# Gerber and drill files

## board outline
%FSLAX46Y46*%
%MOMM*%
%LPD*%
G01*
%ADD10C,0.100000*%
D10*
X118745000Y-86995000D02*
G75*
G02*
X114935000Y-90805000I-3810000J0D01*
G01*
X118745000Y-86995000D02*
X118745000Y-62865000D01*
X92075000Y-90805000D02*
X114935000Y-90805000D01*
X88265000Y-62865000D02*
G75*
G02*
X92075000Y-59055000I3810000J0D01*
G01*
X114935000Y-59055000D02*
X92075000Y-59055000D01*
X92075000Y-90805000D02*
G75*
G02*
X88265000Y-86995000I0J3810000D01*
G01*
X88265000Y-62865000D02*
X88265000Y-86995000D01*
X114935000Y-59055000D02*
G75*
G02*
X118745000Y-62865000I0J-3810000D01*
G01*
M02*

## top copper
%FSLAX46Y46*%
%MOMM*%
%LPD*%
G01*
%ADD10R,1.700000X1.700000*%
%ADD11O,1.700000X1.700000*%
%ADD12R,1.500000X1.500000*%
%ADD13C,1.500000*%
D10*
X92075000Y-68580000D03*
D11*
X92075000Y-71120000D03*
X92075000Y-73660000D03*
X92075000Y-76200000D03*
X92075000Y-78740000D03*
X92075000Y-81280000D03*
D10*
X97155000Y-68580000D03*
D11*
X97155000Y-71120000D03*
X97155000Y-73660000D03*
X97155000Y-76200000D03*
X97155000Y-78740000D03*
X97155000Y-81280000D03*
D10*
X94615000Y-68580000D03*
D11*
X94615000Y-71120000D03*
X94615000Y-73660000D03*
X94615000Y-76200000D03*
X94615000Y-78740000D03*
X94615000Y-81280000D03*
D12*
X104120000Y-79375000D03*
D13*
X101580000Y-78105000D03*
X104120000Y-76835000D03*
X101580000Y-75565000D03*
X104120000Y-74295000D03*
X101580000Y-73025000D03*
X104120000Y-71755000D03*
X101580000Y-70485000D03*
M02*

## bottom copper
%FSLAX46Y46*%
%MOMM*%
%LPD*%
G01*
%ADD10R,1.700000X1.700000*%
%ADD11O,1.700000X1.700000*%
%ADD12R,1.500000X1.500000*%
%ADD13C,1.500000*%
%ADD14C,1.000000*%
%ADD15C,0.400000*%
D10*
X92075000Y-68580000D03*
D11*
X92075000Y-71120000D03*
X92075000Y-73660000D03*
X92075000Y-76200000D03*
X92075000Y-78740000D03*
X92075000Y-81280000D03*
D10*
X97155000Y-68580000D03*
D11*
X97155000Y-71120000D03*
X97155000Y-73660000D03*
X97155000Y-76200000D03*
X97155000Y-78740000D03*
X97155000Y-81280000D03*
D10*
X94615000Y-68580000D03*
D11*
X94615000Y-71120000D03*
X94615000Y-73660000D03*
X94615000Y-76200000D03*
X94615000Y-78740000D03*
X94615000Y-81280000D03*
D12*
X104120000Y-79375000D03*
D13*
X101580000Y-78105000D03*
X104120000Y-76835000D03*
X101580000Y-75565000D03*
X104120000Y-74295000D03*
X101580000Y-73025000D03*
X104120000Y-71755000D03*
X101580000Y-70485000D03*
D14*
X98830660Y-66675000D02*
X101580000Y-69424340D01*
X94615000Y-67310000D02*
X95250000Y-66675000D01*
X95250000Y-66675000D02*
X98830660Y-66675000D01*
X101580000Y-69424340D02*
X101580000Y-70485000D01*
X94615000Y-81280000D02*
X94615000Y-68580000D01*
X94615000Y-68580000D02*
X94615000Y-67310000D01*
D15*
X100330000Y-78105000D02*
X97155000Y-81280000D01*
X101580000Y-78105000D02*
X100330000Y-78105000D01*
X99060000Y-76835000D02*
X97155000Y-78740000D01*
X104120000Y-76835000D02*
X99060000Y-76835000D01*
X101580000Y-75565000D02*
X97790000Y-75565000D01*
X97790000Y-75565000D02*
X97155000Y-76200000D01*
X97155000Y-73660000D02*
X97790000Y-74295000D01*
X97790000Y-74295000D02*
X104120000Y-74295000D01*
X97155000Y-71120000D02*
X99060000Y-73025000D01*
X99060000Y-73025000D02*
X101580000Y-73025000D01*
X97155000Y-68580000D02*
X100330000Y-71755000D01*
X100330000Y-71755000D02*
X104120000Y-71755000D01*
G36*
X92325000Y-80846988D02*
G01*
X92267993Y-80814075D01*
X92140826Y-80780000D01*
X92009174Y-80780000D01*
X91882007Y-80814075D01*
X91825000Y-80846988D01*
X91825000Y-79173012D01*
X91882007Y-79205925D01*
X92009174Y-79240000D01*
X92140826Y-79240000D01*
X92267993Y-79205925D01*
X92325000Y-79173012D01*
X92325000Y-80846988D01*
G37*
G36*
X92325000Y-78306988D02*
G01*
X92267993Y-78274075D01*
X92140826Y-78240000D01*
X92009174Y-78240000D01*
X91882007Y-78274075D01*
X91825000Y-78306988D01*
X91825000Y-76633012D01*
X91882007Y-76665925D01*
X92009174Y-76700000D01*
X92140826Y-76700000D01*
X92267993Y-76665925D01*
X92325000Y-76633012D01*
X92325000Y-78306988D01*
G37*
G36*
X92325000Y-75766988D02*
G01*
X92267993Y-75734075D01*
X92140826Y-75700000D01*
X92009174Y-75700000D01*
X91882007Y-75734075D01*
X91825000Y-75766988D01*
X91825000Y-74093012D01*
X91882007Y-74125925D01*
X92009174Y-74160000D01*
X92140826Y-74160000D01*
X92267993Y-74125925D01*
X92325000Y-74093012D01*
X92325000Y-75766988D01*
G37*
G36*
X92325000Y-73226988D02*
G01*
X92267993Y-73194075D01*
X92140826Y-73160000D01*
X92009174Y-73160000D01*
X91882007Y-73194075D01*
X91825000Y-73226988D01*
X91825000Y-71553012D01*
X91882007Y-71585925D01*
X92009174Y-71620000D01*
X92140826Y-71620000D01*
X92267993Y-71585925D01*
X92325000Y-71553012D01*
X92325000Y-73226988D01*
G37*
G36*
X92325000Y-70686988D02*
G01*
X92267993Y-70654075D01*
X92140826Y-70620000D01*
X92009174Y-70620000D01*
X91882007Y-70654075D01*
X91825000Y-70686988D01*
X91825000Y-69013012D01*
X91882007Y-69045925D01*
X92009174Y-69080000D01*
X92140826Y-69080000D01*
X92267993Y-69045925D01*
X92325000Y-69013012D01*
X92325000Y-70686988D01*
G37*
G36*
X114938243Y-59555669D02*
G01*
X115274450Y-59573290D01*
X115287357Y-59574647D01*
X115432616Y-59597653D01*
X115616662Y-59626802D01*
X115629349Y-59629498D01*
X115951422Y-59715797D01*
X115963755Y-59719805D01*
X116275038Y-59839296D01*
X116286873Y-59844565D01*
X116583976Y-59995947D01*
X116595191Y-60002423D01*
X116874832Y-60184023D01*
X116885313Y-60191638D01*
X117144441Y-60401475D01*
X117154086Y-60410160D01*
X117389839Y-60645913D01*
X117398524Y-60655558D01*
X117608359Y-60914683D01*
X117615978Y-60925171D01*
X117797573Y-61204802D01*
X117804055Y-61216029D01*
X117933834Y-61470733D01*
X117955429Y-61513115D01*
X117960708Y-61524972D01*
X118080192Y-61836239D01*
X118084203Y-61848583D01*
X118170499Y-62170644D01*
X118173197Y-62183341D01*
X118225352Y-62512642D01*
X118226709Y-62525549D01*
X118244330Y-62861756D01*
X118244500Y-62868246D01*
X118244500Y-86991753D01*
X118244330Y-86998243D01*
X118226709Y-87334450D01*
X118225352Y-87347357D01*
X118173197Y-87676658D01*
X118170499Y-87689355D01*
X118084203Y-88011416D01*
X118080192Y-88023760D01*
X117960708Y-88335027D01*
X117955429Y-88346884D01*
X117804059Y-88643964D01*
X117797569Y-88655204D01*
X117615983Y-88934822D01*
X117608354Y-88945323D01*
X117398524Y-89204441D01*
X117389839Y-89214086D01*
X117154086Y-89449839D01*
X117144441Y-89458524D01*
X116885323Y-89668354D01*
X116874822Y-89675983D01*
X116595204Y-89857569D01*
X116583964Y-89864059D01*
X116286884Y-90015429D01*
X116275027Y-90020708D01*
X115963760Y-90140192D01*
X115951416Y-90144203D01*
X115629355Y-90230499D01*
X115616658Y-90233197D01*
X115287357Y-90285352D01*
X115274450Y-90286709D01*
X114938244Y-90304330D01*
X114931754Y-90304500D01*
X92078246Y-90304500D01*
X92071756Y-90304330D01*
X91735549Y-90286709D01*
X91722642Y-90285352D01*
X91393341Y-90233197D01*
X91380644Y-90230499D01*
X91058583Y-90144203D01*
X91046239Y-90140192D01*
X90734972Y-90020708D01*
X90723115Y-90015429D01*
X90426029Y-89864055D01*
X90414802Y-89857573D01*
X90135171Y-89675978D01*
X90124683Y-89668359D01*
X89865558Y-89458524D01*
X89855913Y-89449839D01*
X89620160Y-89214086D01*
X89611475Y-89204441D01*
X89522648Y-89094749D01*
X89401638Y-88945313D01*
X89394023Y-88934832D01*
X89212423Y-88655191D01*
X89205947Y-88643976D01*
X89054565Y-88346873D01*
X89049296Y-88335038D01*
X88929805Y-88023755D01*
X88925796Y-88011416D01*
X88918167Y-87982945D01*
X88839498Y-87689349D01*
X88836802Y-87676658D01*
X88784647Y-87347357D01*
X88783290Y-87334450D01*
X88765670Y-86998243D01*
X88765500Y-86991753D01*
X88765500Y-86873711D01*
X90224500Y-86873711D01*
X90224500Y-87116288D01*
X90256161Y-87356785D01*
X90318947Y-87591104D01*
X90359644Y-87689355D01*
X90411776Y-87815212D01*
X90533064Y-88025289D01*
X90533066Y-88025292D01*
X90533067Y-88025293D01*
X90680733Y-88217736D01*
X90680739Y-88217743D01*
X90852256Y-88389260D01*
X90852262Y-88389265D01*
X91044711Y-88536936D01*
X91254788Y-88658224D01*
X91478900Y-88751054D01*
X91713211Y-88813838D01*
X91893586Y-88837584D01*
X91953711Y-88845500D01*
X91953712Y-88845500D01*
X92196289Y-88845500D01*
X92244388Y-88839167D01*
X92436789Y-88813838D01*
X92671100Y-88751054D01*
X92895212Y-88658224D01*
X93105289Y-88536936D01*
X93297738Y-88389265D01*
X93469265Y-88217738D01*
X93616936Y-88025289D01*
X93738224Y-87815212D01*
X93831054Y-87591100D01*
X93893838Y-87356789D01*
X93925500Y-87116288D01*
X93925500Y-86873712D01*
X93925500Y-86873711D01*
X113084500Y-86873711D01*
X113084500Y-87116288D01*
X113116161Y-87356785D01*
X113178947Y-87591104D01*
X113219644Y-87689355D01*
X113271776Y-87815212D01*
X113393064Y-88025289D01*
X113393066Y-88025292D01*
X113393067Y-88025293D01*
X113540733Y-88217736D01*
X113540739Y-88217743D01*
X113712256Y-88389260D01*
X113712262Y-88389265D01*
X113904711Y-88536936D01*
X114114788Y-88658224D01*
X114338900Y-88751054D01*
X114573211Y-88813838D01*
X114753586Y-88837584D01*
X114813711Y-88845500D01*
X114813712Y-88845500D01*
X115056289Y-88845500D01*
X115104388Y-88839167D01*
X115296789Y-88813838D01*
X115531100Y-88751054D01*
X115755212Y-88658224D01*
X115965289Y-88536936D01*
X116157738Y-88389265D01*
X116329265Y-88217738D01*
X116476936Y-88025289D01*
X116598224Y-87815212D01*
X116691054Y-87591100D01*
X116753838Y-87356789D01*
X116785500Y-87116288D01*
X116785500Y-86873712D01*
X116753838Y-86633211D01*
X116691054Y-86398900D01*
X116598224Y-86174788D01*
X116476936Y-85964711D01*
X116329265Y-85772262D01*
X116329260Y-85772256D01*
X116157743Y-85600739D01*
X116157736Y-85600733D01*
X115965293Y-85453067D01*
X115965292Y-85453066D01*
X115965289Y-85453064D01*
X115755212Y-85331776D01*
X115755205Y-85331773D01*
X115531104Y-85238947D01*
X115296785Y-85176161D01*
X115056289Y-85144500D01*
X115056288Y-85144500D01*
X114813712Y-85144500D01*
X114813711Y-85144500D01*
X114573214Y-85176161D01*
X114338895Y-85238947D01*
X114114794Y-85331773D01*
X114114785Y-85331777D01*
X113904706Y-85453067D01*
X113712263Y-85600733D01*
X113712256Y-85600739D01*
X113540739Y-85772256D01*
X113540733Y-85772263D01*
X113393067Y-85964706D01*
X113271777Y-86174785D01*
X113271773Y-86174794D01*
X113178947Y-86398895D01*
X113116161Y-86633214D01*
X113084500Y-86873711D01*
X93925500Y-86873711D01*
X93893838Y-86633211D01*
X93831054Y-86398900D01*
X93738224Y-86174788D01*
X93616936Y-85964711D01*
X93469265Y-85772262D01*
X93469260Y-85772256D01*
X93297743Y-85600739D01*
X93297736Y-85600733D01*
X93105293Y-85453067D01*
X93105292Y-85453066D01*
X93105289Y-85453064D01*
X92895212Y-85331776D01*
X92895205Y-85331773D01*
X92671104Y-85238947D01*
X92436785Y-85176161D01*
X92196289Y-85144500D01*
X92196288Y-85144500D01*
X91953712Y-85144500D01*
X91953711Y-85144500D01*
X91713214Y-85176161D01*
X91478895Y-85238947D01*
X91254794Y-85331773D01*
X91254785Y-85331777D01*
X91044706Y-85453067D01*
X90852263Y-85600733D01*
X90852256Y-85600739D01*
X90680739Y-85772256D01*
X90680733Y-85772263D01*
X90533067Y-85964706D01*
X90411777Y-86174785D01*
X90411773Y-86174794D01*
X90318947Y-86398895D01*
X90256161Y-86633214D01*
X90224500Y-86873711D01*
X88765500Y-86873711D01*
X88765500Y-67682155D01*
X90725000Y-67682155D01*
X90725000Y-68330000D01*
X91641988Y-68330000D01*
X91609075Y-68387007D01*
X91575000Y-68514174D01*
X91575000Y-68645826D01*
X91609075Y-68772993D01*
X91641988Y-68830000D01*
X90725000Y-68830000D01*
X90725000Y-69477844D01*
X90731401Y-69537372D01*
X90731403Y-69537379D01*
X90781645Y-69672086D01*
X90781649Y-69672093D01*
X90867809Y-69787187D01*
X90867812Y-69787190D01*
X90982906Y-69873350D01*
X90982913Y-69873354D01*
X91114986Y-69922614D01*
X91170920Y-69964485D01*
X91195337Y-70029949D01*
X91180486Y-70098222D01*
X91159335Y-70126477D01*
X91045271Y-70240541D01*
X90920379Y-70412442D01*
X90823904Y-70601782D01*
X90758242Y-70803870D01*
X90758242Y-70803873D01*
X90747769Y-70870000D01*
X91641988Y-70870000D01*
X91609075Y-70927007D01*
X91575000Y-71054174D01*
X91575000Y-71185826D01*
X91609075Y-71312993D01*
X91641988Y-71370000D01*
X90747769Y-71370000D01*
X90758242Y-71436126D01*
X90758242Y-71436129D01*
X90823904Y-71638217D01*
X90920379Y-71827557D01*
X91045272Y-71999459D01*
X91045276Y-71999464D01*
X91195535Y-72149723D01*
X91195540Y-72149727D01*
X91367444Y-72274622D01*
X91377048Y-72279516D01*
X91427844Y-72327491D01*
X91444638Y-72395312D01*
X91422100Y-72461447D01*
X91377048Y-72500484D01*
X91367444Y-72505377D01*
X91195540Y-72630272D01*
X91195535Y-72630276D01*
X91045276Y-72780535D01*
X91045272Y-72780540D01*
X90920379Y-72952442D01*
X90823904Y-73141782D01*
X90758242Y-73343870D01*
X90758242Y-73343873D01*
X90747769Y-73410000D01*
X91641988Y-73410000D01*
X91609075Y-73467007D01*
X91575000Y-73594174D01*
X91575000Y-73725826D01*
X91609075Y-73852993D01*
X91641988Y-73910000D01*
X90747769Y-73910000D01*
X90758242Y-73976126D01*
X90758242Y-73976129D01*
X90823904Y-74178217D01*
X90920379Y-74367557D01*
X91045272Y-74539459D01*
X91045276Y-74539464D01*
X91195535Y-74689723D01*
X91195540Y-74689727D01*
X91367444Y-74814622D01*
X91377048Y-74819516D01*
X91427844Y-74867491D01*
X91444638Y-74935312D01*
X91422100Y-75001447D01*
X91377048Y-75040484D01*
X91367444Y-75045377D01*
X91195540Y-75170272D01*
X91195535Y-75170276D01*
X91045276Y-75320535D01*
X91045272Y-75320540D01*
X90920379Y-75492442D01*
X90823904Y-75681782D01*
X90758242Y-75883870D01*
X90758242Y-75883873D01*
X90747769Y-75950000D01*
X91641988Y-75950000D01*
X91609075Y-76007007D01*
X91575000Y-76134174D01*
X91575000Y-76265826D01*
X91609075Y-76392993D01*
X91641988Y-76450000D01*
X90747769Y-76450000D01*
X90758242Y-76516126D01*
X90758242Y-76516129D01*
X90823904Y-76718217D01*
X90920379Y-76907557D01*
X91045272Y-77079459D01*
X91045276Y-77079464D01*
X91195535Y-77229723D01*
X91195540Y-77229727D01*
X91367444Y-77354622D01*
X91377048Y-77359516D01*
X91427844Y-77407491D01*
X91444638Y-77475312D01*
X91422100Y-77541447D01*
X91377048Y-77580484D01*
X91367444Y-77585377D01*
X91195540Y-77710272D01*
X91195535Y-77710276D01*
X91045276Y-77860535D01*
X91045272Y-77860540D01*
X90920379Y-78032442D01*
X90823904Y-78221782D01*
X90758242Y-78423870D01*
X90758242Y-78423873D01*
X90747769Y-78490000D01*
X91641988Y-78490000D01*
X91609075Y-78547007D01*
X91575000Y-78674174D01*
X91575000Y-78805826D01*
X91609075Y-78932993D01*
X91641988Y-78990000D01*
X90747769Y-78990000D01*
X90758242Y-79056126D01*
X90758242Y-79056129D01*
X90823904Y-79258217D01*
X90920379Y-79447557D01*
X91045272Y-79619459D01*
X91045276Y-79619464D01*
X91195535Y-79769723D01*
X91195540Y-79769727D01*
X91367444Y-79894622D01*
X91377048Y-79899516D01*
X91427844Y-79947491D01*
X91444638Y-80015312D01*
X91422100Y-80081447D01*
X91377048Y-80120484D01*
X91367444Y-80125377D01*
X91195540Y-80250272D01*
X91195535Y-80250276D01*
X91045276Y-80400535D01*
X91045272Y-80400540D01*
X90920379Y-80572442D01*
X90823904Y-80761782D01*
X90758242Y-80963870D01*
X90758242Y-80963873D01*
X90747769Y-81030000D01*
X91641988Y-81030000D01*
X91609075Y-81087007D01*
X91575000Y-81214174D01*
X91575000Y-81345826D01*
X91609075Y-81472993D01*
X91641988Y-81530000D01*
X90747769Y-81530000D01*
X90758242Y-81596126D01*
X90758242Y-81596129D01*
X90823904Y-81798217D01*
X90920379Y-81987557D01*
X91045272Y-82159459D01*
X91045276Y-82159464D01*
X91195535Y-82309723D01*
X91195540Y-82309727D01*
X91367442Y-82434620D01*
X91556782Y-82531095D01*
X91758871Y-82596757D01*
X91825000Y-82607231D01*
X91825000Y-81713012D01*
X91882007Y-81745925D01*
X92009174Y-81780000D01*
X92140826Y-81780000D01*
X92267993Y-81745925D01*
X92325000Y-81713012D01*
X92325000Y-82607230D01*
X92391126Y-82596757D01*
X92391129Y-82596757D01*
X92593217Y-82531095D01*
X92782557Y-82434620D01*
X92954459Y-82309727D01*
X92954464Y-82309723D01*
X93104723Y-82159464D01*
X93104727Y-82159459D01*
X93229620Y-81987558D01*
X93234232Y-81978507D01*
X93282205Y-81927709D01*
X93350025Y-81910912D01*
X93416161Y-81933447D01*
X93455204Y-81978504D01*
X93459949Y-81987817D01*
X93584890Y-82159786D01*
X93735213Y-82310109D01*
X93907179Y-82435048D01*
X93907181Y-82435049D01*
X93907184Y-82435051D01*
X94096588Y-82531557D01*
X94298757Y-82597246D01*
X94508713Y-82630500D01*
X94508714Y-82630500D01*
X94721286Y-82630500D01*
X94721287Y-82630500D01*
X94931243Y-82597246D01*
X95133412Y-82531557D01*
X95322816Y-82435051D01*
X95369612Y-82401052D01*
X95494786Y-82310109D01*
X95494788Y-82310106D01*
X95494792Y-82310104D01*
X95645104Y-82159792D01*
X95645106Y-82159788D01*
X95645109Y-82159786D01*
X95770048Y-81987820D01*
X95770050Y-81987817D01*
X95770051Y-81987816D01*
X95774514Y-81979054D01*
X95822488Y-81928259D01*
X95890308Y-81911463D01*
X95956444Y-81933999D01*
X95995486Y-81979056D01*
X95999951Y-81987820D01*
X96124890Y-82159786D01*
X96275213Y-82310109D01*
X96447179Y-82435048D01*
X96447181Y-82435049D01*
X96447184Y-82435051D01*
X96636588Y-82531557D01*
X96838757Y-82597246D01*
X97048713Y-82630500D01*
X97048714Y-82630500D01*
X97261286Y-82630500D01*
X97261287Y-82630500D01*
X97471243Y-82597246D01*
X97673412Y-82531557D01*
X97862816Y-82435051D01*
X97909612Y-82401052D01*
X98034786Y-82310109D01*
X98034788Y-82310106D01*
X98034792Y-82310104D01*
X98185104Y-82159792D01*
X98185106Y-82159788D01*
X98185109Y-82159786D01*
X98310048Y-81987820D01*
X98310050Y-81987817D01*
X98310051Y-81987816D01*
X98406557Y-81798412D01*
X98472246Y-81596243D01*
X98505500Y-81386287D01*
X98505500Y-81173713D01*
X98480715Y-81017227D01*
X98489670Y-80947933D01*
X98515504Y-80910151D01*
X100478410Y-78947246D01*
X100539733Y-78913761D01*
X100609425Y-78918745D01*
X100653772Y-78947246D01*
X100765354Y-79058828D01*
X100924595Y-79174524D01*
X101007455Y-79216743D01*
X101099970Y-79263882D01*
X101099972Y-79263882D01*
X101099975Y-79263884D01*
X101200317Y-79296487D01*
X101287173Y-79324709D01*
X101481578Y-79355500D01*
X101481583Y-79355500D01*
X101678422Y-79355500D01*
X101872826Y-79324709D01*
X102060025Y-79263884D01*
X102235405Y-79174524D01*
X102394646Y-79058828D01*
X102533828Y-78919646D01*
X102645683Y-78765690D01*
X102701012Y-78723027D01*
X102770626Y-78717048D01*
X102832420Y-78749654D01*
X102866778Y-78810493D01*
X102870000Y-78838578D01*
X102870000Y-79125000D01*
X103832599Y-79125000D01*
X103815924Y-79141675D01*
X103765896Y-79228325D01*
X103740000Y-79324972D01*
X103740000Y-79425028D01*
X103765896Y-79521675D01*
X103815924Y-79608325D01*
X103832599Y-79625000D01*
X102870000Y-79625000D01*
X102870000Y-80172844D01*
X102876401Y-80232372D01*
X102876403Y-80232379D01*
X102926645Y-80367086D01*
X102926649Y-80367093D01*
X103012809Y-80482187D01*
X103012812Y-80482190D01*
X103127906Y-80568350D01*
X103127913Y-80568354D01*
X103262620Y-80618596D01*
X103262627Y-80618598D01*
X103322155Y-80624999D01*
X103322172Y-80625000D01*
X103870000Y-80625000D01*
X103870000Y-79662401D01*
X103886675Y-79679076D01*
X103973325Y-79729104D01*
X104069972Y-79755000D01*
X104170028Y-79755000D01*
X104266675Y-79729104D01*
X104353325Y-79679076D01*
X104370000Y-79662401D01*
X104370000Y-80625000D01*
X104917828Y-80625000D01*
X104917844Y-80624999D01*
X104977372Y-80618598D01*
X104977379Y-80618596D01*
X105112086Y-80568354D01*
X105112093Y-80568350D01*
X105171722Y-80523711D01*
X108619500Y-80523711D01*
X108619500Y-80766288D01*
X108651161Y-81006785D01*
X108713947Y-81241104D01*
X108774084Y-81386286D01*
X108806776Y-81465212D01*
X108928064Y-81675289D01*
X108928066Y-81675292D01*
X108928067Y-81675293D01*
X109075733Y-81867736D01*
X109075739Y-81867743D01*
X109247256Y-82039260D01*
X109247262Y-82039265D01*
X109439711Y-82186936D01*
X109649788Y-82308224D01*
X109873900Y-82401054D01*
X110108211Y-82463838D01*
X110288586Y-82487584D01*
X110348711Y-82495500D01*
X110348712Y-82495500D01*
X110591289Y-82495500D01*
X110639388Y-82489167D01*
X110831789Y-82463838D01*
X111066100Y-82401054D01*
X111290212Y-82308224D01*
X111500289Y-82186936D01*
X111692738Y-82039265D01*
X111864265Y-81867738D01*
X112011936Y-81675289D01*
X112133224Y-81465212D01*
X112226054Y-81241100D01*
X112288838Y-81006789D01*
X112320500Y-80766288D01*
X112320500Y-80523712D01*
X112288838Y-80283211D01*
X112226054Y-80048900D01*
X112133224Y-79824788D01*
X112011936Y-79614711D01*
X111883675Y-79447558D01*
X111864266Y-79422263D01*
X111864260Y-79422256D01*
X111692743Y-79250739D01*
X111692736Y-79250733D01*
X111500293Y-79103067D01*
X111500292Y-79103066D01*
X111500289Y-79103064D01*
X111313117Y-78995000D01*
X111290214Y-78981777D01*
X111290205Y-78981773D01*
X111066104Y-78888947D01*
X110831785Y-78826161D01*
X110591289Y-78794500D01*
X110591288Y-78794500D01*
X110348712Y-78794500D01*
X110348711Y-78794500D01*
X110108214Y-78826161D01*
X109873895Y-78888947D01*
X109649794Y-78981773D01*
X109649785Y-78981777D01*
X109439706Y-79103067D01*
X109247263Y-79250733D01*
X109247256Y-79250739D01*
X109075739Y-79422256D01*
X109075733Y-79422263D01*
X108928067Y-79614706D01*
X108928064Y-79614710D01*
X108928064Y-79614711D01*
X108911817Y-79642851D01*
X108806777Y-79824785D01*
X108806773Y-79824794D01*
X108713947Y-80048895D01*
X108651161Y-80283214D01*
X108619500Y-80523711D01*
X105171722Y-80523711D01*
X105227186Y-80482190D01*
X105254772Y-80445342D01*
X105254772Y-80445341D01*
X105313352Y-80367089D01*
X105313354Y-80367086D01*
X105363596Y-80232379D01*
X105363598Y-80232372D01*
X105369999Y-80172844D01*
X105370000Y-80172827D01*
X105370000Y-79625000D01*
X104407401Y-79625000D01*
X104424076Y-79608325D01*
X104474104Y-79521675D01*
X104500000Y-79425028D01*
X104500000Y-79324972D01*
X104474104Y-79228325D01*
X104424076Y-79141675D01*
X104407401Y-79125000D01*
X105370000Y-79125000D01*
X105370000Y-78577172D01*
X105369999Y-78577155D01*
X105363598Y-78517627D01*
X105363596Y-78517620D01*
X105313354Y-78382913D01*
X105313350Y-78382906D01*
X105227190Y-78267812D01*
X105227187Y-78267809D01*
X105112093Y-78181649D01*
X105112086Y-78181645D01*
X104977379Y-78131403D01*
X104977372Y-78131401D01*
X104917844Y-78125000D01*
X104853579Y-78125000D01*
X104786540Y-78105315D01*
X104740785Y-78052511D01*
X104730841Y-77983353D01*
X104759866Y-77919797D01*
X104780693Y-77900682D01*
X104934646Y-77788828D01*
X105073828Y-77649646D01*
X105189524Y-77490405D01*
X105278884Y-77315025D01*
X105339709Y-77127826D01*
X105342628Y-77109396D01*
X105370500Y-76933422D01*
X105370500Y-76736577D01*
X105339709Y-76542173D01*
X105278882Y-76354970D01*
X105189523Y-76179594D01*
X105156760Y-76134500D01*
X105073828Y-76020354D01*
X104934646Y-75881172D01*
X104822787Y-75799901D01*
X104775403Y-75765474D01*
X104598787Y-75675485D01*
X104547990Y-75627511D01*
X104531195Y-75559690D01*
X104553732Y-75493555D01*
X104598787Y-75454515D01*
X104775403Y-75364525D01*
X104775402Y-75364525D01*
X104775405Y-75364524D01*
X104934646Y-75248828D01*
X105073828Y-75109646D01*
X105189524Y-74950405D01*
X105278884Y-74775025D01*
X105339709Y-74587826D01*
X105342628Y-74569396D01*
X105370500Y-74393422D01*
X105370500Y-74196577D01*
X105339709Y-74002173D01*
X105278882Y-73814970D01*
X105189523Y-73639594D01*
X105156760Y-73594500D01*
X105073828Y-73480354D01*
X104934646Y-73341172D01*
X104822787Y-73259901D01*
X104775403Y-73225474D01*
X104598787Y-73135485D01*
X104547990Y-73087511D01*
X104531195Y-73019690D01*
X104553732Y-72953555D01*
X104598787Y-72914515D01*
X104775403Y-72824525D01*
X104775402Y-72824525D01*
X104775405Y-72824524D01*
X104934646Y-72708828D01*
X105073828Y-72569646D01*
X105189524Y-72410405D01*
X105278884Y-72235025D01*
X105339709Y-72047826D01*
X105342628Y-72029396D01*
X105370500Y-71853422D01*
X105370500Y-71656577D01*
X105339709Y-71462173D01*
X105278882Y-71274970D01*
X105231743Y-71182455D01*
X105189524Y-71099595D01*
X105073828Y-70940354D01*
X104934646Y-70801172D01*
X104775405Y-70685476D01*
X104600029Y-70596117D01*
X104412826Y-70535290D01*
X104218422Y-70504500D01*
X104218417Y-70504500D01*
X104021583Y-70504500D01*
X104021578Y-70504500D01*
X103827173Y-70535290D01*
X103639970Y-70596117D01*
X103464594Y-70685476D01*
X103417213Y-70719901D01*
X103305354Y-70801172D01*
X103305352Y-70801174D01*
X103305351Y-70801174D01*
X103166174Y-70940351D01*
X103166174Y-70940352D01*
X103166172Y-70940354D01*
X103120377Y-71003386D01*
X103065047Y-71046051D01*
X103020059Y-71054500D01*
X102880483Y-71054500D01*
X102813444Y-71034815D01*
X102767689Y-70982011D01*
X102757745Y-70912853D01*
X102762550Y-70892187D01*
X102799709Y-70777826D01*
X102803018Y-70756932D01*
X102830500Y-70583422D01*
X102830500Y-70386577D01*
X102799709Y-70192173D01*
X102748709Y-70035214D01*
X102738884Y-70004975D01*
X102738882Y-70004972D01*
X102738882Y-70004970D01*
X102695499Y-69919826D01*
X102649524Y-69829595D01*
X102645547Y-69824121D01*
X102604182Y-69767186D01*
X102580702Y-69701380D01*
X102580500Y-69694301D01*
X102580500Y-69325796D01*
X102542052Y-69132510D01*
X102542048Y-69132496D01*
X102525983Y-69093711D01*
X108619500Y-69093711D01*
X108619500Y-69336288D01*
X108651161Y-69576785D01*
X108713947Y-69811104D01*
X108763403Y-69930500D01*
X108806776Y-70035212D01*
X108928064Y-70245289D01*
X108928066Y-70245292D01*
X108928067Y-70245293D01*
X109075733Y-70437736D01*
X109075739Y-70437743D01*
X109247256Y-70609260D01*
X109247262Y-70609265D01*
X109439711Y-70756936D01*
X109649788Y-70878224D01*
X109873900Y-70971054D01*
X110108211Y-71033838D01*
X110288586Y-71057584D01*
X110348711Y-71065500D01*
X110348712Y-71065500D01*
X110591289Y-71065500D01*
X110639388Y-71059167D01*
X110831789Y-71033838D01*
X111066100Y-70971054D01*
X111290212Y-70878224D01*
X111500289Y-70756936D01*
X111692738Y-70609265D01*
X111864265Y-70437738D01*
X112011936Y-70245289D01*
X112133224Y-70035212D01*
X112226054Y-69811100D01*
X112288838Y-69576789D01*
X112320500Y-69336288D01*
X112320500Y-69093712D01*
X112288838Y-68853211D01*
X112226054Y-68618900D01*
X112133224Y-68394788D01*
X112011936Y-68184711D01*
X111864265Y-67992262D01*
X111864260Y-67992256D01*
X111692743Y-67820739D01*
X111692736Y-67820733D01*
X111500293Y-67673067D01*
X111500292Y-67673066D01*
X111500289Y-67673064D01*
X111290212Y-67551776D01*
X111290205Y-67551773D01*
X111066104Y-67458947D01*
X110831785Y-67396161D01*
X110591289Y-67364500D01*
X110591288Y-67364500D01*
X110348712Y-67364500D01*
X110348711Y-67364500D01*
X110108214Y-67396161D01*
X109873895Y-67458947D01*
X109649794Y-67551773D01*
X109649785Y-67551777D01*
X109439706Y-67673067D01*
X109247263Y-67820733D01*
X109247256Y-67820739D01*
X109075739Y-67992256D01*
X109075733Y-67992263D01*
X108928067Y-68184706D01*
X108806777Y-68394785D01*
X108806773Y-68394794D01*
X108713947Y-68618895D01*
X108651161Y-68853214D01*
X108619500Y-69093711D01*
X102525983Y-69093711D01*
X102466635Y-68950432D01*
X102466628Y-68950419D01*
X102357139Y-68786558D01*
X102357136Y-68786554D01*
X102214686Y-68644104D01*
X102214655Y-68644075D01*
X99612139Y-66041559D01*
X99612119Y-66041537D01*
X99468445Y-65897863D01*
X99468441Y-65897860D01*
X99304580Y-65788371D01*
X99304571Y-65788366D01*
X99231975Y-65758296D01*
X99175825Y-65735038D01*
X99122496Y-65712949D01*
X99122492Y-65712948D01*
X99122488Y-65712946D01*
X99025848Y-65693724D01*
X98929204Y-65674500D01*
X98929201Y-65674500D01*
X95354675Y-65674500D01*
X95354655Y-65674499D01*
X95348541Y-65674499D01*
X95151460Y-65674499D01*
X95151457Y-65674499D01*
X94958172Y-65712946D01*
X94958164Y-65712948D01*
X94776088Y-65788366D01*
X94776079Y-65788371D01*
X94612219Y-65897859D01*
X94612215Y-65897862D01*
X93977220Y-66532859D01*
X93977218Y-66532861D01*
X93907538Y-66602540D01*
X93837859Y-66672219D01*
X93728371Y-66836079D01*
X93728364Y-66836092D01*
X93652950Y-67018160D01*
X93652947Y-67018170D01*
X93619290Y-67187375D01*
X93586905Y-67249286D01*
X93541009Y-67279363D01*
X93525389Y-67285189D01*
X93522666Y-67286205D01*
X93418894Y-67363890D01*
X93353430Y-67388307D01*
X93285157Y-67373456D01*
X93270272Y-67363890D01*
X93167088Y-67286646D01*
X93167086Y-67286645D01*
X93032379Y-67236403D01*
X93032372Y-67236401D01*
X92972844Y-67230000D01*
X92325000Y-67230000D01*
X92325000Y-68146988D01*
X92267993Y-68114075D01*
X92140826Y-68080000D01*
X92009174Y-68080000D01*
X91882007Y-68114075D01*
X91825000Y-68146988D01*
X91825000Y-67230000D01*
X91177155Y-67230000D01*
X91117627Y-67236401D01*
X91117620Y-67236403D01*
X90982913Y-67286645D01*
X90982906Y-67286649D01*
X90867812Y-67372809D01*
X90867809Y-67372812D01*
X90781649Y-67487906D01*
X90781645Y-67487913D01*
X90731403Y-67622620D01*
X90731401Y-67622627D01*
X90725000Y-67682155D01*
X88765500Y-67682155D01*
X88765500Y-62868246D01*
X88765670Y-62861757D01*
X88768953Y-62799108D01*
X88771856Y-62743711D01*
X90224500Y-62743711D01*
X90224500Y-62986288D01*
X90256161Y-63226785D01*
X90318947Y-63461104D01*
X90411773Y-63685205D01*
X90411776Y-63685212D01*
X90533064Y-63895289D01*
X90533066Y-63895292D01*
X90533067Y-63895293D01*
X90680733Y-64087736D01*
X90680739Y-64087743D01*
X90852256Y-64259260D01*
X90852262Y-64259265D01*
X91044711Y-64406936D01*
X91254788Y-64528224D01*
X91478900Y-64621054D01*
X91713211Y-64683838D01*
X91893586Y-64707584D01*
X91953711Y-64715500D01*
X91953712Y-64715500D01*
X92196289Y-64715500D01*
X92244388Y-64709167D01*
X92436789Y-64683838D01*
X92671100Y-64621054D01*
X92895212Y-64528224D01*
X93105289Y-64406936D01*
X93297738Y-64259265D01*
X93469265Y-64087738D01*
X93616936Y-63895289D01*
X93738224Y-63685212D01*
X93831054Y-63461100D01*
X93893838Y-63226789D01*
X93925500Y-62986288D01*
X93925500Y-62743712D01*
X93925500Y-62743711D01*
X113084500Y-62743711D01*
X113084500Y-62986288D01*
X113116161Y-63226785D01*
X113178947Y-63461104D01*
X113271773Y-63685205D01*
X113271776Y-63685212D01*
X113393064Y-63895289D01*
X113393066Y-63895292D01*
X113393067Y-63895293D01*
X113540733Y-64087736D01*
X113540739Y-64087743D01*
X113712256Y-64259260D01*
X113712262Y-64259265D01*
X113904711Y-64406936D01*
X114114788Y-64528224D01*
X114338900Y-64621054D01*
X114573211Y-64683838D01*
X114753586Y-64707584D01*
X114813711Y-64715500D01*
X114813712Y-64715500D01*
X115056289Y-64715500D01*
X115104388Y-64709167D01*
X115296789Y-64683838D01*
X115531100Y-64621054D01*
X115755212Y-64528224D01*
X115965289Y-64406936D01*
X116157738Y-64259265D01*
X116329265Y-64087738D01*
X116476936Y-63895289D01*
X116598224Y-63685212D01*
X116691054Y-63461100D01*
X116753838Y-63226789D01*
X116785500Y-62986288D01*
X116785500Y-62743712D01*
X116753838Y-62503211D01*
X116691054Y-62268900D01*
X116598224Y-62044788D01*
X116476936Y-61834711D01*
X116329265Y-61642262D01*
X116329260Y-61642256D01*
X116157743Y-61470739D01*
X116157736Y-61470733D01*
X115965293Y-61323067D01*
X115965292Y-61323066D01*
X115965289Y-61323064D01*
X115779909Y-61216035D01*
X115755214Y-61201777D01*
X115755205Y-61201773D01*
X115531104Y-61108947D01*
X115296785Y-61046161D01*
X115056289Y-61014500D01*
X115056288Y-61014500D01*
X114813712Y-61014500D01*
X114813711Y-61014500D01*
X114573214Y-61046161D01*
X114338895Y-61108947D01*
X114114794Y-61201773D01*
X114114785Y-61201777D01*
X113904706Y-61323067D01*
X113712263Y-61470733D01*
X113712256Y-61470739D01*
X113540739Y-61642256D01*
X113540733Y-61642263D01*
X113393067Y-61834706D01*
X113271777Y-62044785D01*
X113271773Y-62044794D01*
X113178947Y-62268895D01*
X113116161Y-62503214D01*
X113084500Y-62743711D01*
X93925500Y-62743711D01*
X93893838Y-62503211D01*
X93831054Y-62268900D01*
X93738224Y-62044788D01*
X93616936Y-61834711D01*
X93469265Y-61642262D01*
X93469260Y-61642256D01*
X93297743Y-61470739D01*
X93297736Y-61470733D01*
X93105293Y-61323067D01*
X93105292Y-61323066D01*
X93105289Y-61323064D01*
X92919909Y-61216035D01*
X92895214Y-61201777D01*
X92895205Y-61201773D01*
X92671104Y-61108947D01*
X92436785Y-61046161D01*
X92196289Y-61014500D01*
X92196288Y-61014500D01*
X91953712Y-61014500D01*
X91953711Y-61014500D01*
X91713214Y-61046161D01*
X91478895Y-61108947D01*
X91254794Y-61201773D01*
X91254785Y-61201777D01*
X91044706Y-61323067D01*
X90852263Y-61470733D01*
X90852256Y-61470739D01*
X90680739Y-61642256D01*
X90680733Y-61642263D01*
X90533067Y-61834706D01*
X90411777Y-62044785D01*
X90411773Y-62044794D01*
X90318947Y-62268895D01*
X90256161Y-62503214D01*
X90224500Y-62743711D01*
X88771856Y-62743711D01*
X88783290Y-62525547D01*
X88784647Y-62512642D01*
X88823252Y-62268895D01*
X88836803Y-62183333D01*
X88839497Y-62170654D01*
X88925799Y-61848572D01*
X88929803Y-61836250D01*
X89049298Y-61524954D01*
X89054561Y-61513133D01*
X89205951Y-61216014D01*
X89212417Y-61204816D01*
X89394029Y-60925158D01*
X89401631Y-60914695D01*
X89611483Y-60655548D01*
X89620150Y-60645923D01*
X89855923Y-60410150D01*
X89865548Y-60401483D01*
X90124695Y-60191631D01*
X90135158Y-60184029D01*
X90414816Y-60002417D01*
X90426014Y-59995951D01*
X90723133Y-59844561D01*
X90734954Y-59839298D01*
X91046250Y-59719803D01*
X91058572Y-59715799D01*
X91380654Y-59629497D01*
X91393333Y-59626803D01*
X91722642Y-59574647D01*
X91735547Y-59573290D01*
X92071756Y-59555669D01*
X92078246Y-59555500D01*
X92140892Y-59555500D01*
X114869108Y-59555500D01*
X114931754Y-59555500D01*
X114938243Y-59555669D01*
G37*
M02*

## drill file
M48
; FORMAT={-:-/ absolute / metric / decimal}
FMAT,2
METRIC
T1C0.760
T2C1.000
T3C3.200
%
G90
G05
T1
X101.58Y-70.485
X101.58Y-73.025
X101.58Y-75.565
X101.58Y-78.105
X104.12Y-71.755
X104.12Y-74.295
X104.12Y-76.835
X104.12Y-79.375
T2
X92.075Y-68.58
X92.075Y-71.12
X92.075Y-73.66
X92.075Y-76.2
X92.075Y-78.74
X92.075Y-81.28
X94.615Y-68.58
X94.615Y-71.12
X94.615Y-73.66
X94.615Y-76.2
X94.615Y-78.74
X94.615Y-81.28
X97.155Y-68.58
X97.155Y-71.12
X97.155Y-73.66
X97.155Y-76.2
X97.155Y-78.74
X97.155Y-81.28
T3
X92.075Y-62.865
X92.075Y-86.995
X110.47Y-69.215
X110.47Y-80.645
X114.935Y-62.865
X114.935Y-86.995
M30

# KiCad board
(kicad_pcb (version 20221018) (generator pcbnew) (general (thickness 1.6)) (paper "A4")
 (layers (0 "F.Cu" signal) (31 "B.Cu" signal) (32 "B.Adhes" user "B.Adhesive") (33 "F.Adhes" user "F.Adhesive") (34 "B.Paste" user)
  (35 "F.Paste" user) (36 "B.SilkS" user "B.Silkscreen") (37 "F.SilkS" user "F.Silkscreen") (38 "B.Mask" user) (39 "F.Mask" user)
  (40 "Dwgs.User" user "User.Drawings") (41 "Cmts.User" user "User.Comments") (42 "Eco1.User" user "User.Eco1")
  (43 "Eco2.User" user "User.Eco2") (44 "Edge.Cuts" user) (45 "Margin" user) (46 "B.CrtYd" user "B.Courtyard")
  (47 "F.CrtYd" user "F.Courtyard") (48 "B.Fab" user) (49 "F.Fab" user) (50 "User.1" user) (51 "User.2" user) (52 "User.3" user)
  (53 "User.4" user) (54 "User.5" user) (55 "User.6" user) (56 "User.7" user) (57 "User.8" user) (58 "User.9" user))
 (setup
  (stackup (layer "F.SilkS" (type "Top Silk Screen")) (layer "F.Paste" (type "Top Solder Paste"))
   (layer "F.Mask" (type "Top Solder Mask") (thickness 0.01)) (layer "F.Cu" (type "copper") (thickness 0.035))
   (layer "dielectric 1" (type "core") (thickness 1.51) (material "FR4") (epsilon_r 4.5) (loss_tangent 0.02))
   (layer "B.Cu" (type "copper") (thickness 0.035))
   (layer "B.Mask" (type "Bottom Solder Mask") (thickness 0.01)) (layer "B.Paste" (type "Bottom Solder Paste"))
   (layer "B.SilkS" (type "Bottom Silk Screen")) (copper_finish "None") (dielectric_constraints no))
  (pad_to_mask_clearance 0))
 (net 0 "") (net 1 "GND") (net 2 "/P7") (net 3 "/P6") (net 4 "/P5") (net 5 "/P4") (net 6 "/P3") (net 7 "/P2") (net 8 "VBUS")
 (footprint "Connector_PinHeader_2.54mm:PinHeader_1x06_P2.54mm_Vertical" (layer "F.Cu") (at 92.075 68.58)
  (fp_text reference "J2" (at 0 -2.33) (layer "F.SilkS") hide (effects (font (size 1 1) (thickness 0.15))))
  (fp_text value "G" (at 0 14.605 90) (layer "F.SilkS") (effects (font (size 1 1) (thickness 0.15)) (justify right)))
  (pad "1" thru_hole rect (at 0 0) (size 1.7 1.7) (drill 1) (layers "*.Cu" "*.Mask") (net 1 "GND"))
  (pad "2" thru_hole oval (at 0 2.54) (size 1.7 1.7) (drill 1) (layers "*.Cu" "*.Mask") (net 1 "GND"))
  (pad "3" thru_hole oval (at 0 5.08) (size 1.7 1.7) (drill 1) (layers "*.Cu" "*.Mask") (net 1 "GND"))
  (pad "4" thru_hole oval (at 0 7.62) (size 1.7 1.7) (drill 1) (layers "*.Cu" "*.Mask") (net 1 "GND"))
  (pad "5" thru_hole oval (at 0 10.16) (size 1.7 1.7) (drill 1) (layers "*.Cu" "*.Mask") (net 1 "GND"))
  (pad "6" thru_hole oval (at 0 12.7) (size 1.7 1.7) (drill 1) (layers "*.Cu" "*.Mask") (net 1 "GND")))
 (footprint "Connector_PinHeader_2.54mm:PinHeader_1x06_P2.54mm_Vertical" (layer "F.Cu") (at 97.155 68.58)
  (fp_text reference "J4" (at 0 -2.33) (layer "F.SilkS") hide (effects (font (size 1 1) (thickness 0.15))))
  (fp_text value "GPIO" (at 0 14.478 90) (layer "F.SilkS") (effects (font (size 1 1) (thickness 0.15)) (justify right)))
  (pad "1" thru_hole rect (at 0 0) (size 1.7 1.7) (drill 1) (layers "*.Cu" "*.Mask") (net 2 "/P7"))
  (pad "2" thru_hole oval (at 0 2.54) (size 1.7 1.7) (drill 1) (layers "*.Cu" "*.Mask") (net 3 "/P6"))
  (pad "3" thru_hole oval (at 0 5.08) (size 1.7 1.7) (drill 1) (layers "*.Cu" "*.Mask") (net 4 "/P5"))
  (pad "4" thru_hole oval (at 0 7.62) (size 1.7 1.7) (drill 1) (layers "*.Cu" "*.Mask") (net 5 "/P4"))
  (pad "5" thru_hole oval (at 0 10.16) (size 1.7 1.7) (drill 1) (layers "*.Cu" "*.Mask") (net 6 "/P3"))
  (pad "6" thru_hole oval (at 0 12.7) (size 1.7 1.7) (drill 1) (layers "*.Cu" "*.Mask") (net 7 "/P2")))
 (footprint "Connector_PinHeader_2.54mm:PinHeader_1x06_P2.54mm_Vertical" (layer "F.Cu") (at 94.615 68.58)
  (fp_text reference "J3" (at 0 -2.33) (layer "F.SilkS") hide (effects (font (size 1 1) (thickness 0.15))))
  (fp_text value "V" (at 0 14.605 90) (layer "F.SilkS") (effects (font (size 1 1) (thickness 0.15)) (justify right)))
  (pad "1" thru_hole rect (at 0 0) (size 1.7 1.7) (drill 1) (layers "*.Cu" "*.Mask") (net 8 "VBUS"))
  (pad "2" thru_hole oval (at 0 2.54) (size 1.7 1.7) (drill 1) (layers "*.Cu" "*.Mask") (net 8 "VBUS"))
  (pad "3" thru_hole oval (at 0 5.08) (size 1.7 1.7) (drill 1) (layers "*.Cu" "*.Mask") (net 8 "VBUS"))
  (pad "4" thru_hole oval (at 0 7.62) (size 1.7 1.7) (drill 1) (layers "*.Cu" "*.Mask") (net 8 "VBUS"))
  (pad "5" thru_hole oval (at 0 10.16) (size 1.7 1.7) (drill 1) (layers "*.Cu" "*.Mask") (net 8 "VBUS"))
  (pad "6" thru_hole oval (at 0 12.7) (size 1.7 1.7) (drill 1) (layers "*.Cu" "*.Mask") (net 8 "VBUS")))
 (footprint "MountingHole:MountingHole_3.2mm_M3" (layer "F.Cu") (at 92.075 62.865)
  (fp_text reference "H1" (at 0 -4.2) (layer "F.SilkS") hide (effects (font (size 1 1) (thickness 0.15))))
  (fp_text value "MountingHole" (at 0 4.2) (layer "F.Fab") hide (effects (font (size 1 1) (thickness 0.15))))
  (pad "" np_thru_hole circle (at 0 0) (size 3.2 3.2) (drill 3.2) (layers "*.Cu" "*.Mask")))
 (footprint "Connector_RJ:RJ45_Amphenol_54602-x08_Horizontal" (layer "F.Cu") (at 104.12 79.375 90)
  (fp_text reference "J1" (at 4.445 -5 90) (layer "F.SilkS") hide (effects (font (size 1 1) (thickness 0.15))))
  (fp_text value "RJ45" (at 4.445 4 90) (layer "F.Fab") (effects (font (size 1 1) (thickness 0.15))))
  (pad "" np_thru_hole circle (at -1.27 6.35 90) (size 3.2 3.2) (drill 3.2) (layers "*.Cu" "*.Mask"))
  (pad "" np_thru_hole circle (at 10.16 6.35 90) (size 3.2 3.2) (drill 3.2) (layers "*.Cu" "*.Mask"))
  (pad "1" thru_hole rect (at 0 0 90) (size 1.5 1.5) (drill 0.76) (layers "*.Cu" "*.Mask") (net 1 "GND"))
  (pad "2" thru_hole circle (at 1.27 -2.54 90) (size 1.5 1.5) (drill 0.76) (layers "*.Cu" "*.Mask") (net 7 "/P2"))
  (pad "3" thru_hole circle (at 2.54 0 90) (size 1.5 1.5) (drill 0.76) (layers "*.Cu" "*.Mask") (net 6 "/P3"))
  (pad "4" thru_hole circle (at 3.81 -2.54 90) (size 1.5 1.5) (drill 0.76) (layers "*.Cu" "*.Mask") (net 5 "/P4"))
  (pad "5" thru_hole circle (at 5.08 0 90) (size 1.5 1.5) (drill 0.76) (layers "*.Cu" "*.Mask") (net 4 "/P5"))
  (pad "6" thru_hole circle (at 6.35 -2.54 90) (size 1.5 1.5) (drill 0.76) (layers "*.Cu" "*.Mask") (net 3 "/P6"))
  (pad "7" thru_hole circle (at 7.62 0 90) (size 1.5 1.5) (drill 0.76) (layers "*.Cu" "*.Mask") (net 2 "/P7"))
  (pad "8" thru_hole circle (at 8.89 -2.54 90) (size 1.5 1.5) (drill 0.76) (layers "*.Cu" "*.Mask") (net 8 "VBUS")))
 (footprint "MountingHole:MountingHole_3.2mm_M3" (layer "F.Cu") (at 114.935 62.865)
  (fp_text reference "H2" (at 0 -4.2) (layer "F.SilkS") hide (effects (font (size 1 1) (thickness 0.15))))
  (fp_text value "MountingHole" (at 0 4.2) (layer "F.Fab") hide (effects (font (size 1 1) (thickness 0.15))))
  (pad "" np_thru_hole circle (at 0 0) (size 3.2 3.2) (drill 3.2) (layers "*.Cu" "*.Mask")))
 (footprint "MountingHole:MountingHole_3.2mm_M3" (layer "F.Cu") (at 92.075 86.995)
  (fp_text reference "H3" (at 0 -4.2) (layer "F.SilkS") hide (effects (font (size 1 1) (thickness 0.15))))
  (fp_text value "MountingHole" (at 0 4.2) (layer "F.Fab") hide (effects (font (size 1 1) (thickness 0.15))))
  (pad "" np_thru_hole circle (at 0 0) (size 3.2 3.2) (drill 3.2) (layers "*.Cu" "*.Mask")))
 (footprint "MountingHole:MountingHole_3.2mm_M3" (layer "F.Cu") (at 114.935 86.995)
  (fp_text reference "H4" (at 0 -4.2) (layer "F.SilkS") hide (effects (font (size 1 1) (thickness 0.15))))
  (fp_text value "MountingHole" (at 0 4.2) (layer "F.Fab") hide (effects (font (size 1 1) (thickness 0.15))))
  (pad "" np_thru_hole circle (at 0 0) (size 3.2 3.2) (drill 3.2) (layers "*.Cu" "*.Mask")))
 (gr_arc (start 118.745 86.995) (mid 117.629077 89.689077) (end 114.935 90.805) (stroke (width 0.1) (type default)) (layer "Edge.Cuts"))
 (gr_line (start 118.745 86.995) (end 118.745 62.865) (stroke (width 0.1) (type default)) (layer "Edge.Cuts"))
 (gr_line (start 92.075 90.805) (end 114.935 90.805) (stroke (width 0.1) (type default)) (layer "Edge.Cuts"))
 (gr_arc (start 88.265 62.865) (mid 89.380923 60.170923) (end 92.075 59.055) (stroke (width 0.1) (type default)) (layer "Edge.Cuts"))
 (gr_line (start 114.935 59.055) (end 92.075 59.055) (stroke (width 0.1) (type default)) (layer "Edge.Cuts"))
 (gr_arc (start 92.075 90.805) (mid 89.380923 89.689077) (end 88.265 86.995) (stroke (width 0.1) (type default)) (layer "Edge.Cuts"))
 (gr_line (start 88.265 62.865) (end 88.265 86.995) (stroke (width 0.1) (type default)) (layer "Edge.Cuts"))
 (gr_arc (start 114.935 59.055) (mid 117.629077 60.170923) (end 118.745 62.865) (stroke (width 0.1) (type default)) (layer "Edge.Cuts"))
 (segment (start 98.83066 66.675) (end 101.58 69.42434) (width 1) (layer "B.Cu") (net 8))
 (segment (start 94.615 67.31) (end 95.25 66.675) (width 1) (layer "B.Cu") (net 8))
 (segment (start 95.25 66.675) (end 98.83066 66.675) (width 1) (layer "B.Cu") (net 8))
 (segment (start 101.58 69.42434) (end 101.58 70.485) (width 1) (layer "B.Cu") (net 8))
 (segment (start 94.615 81.28) (end 94.615 68.58) (width 1) (layer "B.Cu") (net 8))
 (segment (start 94.615 68.58) (end 94.615 67.31) (width 1) (layer "B.Cu") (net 8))
 (segment (start 100.33 78.105) (end 97.155 81.28) (width 0.4) (layer "B.Cu") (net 7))
 (segment (start 101.58 78.105) (end 100.33 78.105) (width 0.4) (layer "B.Cu") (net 7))
 (segment (start 99.06 76.835) (end 97.155 78.74) (width 0.4) (layer "B.Cu") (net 6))
 (segment (start 104.12 76.835) (end 99.06 76.835) (width 0.4) (layer "B.Cu") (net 6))
 (segment (start 101.58 75.565) (end 97.79 75.565) (width 0.4) (layer "B.Cu") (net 5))
 (segment (start 97.79 75.565) (end 97.155 76.2) (width 0.4) (layer "B.Cu") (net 5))
 (segment (start 97.155 73.66) (end 97.79 74.295) (width 0.4) (layer "B.Cu") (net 4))
 (segment (start 97.79 74.295) (end 104.12 74.295) (width 0.4) (layer "B.Cu") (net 4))
 (segment (start 97.155 71.12) (end 99.06 73.025) (width 0.4) (layer "B.Cu") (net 3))
 (segment (start 99.06 73.025) (end 101.58 73.025) (width 0.4) (layer "B.Cu") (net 3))
 (segment (start 97.155 68.58) (end 100.33 71.755) (width 0.4) (layer "B.Cu") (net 2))
 (segment (start 100.33 71.755) (end 104.12 71.755) (width 0.4) (layer "B.Cu") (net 2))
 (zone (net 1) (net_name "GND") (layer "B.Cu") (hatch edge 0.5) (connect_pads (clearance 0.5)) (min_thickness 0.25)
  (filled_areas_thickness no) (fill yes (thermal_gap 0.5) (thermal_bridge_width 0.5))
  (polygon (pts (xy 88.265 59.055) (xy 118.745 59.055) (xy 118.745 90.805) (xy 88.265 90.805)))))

